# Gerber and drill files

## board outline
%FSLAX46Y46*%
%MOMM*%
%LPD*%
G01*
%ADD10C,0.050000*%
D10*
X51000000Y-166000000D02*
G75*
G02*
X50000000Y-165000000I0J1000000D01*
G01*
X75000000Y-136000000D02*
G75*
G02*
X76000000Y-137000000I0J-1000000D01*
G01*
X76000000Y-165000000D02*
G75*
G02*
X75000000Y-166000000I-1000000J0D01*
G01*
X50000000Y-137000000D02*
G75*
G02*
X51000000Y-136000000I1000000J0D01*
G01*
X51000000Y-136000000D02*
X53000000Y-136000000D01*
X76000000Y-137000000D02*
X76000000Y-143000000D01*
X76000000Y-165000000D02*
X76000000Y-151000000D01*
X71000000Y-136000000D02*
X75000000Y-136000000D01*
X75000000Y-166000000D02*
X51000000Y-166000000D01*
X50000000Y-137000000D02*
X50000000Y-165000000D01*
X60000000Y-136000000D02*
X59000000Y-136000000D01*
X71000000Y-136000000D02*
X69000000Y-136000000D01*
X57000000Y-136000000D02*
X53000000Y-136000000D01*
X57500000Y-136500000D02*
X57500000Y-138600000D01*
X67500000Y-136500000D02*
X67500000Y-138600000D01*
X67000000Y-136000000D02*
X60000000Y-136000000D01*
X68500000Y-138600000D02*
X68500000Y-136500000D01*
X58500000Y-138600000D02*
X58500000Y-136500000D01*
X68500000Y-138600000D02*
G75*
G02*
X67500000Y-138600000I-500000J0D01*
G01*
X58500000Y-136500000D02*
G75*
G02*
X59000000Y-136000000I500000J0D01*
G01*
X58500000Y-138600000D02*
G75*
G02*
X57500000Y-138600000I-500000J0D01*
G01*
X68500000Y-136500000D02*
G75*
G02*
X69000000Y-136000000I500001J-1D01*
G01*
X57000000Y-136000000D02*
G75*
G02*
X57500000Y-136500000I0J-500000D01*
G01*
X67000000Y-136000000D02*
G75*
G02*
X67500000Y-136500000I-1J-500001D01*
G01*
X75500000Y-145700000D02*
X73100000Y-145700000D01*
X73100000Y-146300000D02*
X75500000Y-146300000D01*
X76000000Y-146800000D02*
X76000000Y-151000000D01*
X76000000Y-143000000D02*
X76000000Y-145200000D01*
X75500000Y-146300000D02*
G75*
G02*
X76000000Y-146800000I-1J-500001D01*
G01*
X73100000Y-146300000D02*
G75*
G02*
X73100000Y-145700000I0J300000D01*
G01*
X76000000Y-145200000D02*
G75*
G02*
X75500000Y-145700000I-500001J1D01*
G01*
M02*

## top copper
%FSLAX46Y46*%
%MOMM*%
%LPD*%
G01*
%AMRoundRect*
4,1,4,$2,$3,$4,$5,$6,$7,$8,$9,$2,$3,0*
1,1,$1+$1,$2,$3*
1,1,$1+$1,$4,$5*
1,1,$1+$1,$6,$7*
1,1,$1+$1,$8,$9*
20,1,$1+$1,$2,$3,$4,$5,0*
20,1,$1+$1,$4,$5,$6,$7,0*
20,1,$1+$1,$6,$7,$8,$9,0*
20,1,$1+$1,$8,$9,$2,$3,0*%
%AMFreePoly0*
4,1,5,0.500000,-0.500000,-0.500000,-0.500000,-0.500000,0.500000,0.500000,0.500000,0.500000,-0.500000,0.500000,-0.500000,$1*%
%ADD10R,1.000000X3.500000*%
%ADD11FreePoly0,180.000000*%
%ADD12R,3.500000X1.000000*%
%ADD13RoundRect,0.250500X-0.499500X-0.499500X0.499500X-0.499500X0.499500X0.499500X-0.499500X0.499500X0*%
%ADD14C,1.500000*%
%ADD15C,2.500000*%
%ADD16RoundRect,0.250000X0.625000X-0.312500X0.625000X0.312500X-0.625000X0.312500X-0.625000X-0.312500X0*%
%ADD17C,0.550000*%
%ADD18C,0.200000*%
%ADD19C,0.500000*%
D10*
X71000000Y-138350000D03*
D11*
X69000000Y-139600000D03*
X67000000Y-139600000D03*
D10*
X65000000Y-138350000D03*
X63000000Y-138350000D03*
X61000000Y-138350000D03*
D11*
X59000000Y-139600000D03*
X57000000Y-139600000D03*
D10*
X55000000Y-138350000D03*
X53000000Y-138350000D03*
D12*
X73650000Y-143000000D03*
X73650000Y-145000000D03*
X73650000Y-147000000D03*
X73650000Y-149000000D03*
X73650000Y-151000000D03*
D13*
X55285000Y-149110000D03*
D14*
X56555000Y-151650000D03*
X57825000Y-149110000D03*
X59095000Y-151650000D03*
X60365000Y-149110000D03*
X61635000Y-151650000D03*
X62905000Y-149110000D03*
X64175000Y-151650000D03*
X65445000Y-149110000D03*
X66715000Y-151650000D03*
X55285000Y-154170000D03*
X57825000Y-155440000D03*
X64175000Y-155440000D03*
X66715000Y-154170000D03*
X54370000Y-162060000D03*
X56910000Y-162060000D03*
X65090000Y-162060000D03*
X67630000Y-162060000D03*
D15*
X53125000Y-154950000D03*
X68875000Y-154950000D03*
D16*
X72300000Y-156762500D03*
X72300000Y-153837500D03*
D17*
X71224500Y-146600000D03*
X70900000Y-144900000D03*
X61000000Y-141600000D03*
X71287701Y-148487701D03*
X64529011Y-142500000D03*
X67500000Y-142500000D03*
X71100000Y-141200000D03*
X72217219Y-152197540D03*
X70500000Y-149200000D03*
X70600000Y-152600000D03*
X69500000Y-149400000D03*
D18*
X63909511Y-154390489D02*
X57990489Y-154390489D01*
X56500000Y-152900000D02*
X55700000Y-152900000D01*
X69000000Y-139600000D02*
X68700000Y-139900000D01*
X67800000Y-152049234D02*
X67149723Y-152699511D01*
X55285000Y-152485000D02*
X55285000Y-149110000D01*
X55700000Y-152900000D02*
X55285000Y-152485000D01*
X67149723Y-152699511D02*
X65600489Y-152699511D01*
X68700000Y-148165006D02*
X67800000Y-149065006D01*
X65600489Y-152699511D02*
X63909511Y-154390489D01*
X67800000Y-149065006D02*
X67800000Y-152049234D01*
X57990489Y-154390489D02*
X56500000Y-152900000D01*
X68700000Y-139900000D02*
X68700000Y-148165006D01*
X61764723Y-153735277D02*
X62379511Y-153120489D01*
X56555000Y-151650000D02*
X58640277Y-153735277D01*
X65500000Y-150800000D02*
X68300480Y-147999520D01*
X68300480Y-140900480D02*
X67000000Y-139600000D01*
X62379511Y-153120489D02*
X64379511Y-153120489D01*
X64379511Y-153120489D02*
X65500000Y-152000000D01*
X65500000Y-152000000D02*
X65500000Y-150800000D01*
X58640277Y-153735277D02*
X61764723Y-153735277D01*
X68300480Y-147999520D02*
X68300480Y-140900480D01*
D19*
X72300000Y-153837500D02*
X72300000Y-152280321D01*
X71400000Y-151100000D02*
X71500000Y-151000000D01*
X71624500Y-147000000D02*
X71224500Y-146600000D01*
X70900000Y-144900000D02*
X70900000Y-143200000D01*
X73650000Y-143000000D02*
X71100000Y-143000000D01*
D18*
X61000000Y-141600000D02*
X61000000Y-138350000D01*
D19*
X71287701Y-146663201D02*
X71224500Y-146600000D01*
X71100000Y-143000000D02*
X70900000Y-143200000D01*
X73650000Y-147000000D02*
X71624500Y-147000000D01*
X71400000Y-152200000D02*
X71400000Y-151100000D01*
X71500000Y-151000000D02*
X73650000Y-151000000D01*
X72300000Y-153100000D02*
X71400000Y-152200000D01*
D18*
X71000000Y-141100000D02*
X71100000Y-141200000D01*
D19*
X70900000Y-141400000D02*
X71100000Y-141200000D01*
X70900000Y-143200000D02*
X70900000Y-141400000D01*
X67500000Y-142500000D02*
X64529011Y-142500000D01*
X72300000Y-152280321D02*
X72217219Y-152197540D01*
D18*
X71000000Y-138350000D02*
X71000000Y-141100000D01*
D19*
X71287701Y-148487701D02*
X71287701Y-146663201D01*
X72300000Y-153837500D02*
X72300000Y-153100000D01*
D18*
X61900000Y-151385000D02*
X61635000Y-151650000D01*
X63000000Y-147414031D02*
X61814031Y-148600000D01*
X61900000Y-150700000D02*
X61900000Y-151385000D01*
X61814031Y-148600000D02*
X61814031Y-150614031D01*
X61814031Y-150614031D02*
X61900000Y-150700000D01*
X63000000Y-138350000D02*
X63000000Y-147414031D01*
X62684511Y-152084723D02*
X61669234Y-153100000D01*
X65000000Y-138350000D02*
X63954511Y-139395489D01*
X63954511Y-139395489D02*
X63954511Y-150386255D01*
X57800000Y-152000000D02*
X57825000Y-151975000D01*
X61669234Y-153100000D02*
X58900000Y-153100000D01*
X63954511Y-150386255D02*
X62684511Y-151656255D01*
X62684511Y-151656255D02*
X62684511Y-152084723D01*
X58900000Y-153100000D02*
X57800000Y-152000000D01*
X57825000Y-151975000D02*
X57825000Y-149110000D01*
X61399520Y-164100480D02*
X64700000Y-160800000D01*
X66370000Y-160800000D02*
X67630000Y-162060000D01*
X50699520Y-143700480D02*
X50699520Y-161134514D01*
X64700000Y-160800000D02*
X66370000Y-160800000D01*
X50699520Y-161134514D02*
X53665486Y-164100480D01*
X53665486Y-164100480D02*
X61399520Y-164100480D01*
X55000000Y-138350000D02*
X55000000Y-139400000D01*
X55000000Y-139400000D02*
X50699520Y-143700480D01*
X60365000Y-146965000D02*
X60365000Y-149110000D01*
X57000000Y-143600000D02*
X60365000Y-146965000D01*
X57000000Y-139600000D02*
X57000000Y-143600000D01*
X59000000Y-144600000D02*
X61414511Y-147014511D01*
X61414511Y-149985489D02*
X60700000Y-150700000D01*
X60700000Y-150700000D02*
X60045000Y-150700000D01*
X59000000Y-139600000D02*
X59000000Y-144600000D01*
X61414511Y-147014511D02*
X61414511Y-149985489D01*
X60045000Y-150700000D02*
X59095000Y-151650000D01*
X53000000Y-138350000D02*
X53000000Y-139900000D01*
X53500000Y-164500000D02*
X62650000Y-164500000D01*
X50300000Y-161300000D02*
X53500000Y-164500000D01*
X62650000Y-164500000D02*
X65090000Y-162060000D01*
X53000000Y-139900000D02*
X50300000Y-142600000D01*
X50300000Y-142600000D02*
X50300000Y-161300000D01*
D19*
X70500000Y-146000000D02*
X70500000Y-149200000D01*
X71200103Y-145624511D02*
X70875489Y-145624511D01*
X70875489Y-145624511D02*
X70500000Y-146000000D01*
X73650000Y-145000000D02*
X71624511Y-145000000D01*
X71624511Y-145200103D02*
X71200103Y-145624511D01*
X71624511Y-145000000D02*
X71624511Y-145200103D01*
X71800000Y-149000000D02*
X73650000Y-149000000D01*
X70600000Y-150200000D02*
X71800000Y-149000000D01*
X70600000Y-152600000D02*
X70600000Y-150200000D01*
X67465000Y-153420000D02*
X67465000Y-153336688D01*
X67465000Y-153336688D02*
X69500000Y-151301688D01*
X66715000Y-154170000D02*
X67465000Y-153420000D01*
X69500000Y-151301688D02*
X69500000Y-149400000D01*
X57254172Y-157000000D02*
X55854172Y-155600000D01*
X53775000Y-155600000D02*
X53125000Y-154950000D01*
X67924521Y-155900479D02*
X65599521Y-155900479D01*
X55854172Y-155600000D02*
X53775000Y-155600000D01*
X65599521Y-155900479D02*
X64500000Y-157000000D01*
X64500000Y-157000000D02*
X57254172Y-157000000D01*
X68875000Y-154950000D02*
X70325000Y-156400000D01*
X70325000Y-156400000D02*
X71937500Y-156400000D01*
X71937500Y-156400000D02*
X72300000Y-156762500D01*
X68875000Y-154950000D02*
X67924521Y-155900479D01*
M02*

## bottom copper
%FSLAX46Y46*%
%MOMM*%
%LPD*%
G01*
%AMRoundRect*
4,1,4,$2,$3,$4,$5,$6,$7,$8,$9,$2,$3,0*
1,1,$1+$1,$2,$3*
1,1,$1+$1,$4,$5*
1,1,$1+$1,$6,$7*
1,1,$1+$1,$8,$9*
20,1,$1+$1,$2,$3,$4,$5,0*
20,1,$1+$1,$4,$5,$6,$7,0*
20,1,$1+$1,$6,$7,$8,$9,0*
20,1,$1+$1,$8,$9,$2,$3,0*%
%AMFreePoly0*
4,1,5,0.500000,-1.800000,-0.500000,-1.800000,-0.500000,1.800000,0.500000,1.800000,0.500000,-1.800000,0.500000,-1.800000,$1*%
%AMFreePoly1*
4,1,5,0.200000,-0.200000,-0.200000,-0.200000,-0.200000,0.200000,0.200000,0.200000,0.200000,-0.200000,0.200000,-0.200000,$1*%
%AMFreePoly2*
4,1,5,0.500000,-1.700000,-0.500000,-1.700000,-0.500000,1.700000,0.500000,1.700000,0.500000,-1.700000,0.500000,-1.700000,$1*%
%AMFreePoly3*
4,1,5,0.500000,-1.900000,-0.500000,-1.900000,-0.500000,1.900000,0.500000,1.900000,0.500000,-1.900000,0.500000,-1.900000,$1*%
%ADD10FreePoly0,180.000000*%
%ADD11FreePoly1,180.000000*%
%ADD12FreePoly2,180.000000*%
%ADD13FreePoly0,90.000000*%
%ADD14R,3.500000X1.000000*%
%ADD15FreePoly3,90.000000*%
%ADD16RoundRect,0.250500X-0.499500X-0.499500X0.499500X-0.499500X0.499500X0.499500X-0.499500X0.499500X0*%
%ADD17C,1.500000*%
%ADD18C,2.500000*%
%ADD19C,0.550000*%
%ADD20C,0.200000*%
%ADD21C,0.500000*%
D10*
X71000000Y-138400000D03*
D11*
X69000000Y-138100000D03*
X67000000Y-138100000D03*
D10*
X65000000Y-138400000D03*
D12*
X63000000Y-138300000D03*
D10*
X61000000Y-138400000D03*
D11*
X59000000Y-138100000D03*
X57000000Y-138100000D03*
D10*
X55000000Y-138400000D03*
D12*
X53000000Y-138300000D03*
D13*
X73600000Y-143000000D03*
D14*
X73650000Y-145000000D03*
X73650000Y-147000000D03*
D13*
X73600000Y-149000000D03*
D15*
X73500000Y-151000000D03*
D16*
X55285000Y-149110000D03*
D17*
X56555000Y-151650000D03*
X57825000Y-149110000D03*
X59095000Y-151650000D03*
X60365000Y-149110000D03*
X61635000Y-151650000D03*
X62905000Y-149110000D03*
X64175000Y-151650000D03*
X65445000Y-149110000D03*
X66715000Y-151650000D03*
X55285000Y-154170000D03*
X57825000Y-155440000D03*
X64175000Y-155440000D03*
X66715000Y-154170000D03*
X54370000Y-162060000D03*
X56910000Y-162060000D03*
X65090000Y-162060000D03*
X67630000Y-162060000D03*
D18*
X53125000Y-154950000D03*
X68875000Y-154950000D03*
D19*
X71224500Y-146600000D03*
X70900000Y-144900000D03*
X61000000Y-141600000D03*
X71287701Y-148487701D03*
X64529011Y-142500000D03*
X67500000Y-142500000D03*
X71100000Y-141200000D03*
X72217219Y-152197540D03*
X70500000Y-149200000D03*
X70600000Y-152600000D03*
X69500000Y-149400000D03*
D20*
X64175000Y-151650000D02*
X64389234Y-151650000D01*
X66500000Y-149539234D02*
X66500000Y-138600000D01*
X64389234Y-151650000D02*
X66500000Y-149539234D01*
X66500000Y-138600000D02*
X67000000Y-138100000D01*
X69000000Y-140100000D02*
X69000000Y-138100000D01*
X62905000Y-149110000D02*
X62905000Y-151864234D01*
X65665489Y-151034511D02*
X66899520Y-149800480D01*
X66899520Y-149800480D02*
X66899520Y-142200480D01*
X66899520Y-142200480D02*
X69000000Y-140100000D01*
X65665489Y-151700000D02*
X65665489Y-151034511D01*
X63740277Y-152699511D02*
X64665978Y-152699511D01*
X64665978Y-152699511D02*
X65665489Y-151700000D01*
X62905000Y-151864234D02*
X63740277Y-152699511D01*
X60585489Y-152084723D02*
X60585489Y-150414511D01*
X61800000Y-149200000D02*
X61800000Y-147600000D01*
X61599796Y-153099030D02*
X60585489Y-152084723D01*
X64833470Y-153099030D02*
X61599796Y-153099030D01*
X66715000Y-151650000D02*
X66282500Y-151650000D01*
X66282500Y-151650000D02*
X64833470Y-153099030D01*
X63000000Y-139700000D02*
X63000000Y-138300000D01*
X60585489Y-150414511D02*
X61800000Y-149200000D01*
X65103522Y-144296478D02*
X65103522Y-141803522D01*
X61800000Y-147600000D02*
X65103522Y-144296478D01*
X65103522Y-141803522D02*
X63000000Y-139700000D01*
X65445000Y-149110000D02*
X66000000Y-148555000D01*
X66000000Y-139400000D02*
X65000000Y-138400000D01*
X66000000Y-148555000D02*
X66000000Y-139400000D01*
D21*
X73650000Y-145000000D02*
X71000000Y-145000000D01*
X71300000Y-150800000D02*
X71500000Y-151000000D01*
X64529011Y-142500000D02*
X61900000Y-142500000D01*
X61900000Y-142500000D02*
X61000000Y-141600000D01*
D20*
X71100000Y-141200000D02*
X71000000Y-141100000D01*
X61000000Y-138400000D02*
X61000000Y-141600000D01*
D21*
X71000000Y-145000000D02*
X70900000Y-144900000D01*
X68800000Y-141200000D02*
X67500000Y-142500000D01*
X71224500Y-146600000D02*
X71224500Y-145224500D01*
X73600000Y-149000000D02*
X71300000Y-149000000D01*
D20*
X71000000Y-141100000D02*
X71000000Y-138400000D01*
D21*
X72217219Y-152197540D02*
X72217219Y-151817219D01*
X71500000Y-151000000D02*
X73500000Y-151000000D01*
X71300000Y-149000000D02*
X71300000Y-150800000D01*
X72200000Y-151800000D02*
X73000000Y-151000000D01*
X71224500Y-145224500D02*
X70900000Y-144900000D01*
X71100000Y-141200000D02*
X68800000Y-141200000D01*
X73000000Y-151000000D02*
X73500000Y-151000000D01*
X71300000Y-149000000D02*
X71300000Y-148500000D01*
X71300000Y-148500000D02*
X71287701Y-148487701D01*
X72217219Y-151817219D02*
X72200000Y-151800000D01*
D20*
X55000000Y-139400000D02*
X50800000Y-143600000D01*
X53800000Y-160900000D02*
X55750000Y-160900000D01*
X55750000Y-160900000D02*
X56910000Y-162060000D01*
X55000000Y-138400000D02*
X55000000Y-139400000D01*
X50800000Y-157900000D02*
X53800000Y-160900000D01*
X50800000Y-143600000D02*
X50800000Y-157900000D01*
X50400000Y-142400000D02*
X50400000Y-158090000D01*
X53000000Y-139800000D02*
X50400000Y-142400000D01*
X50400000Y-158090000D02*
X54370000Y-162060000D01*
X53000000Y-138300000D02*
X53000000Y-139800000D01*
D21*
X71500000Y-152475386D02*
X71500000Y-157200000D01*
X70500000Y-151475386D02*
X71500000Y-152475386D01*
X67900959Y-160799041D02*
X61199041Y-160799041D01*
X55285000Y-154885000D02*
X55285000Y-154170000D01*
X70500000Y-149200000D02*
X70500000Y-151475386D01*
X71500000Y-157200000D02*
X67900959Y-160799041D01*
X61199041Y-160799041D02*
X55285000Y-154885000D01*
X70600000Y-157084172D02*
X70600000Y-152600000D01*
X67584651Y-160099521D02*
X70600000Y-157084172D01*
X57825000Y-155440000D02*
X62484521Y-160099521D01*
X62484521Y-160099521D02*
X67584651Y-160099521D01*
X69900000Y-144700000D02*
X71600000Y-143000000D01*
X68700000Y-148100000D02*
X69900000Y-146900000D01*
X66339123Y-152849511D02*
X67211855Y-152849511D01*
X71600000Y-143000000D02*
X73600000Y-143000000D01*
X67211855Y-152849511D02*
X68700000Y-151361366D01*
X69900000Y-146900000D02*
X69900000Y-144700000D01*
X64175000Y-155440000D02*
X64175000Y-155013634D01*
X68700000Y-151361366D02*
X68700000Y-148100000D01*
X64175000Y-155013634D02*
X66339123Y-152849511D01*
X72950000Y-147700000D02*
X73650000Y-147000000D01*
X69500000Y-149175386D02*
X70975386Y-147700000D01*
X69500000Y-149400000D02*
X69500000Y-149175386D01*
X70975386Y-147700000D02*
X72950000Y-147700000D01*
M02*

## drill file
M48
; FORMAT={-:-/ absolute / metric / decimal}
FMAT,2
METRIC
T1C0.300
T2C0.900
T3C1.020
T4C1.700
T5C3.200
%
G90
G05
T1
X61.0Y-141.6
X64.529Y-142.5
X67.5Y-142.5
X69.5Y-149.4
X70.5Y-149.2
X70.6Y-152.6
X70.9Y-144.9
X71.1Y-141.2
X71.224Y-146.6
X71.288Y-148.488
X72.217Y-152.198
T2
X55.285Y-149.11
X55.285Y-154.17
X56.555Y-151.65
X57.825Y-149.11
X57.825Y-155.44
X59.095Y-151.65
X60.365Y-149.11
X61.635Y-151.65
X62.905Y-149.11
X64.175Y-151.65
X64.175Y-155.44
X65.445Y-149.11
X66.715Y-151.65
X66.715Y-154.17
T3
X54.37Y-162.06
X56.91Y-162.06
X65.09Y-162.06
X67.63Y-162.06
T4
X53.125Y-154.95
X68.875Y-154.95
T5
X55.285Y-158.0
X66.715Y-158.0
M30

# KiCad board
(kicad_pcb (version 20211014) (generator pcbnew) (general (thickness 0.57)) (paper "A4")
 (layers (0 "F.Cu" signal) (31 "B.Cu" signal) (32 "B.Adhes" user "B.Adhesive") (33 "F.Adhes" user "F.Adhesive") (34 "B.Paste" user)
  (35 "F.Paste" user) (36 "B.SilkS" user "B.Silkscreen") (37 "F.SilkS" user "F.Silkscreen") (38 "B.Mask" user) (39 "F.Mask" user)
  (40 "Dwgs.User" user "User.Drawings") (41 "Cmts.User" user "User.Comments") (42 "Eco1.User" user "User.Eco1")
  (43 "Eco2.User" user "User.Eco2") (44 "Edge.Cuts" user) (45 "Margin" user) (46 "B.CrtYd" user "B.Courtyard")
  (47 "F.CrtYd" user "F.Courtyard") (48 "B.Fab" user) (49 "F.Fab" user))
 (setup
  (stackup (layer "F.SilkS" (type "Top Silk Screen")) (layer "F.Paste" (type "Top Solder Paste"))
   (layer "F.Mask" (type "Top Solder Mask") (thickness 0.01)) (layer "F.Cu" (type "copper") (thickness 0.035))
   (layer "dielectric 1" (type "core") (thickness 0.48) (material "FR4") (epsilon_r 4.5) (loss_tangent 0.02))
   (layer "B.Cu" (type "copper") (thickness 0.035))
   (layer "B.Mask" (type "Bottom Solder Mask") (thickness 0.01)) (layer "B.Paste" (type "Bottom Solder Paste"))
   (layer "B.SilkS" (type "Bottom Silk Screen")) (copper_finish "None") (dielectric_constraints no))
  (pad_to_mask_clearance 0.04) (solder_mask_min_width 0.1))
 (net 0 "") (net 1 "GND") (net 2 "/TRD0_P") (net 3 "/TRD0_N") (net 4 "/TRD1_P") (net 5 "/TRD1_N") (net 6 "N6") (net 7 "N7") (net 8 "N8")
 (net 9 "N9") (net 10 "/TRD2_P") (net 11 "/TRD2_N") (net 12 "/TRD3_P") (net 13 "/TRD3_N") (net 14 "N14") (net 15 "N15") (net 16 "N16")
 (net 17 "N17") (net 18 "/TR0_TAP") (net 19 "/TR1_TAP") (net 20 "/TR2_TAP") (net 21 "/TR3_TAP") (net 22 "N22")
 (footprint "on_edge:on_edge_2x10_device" (layer "F.Cu") (at 67 136 180)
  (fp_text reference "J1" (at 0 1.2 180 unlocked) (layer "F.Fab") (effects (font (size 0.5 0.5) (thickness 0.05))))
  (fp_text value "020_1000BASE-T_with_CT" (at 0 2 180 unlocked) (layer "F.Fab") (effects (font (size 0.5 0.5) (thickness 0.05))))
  (fp_line (start 7 0) (end 8 0) (layer "Edge.Cuts") (width 0.05))
  (fp_line (start -4 0) (end -2 0) (layer "Edge.Cuts") (width 0.05))
  (fp_line (start 10 0) (end 14 0) (layer "Edge.Cuts") (width 0.05))
  (fp_line (start 9.5 -0.5) (end 9.5 -2.6) (layer "Edge.Cuts") (width 0.05))
  (fp_line (start -0.5 -0.5) (end -0.5 -2.6) (layer "Edge.Cuts") (width 0.05))
  (fp_line (start 0 0) (end 7 0) (layer "Edge.Cuts") (width 0.05))
  (fp_line (start -1.5 -2.6) (end -1.5 -0.5) (layer "Edge.Cuts") (width 0.05))
  (fp_line (start 8.5 -2.6) (end 8.5 -0.5) (layer "Edge.Cuts") (width 0.05))
  (fp_arc (start -1.5 -2.6) (mid -1 -3.1) (end -0.5 -2.6) (layer "Edge.Cuts") (width 0.05))
  (fp_arc (start 8.5 -0.5) (mid 8.353553 -0.146447) (end 8 0) (layer "Edge.Cuts") (width 0.05))
  (fp_arc (start 8.5 -2.6) (mid 9 -3.1) (end 9.5 -2.6) (layer "Edge.Cuts") (width 0.05))
  (fp_arc (start -1.5 -0.5) (mid -1.646447 -0.146447) (end -2 0) (layer "Edge.Cuts") (width 0.05))
  (fp_arc (start 10 0) (mid 9.646447 -0.146447) (end 9.5 -0.5) (layer "Edge.Cuts") (width 0.05))
  (fp_arc (start 0 0) (mid -0.353553 -0.146447) (end -0.5 -0.5) (layer "Edge.Cuts") (width 0.05))
  (pad "1" smd rect locked (at -4 -2.35) (size 1 3.5) (layers "F.Cu" "F.Mask") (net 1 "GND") (zone_connect 0))
  (pad "2" smd custom locked (at -2 -3.6 180) (size 1 1) (layers "F.Cu" "F.Mask") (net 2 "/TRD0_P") (zone_connect 0)
   (options (clearance outline) (anchor rect)) (primitives))
  (pad "3" smd custom locked (at 0 -3.6 180) (size 1 1) (layers "F.Cu" "F.Mask") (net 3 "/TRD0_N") (zone_connect 0)
   (options (clearance outline) (anchor rect)) (primitives))
  (pad "4" smd rect locked (at 2 -2.35) (size 1 3.5) (layers "F.Cu" "F.Mask") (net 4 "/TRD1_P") (zone_connect 0))
  (pad "5" smd rect locked (at 4 -2.35) (size 1 3.5) (layers "F.Cu" "F.Mask") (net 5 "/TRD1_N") (zone_connect 0))
  (pad "6" smd rect locked (at 6 -2.35) (size 1 3.5) (layers "F.Cu" "F.Mask") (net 1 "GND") (zone_connect 0))
  (pad "7" smd custom locked (at 8 -3.6 180) (size 1 1) (layers "F.Cu" "F.Mask") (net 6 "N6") (zone_connect 0)
   (options (clearance outline) (anchor rect)) (primitives))
  (pad "8" smd custom locked (at 10 -3.6 180) (size 1 1) (layers "F.Cu" "F.Mask") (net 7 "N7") (zone_connect 0)
   (options (clearance outline) (anchor rect)) (primitives))
  (pad "9" smd rect locked (at 12 -2.35) (size 1 3.5) (layers "F.Cu" "F.Mask") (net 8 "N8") (zone_connect 0))
  (pad "10" smd rect locked (at 14 -2.35) (size 1 3.5) (layers "F.Cu" "F.Mask") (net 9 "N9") (zone_connect 0))
  (pad "11" smd custom locked (at -4 -2.4 180) (size 1 3.6) (layers "B.Cu" "B.Mask") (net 1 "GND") (zone_connect 0)
   (options (clearance outline) (anchor rect)) (primitives))
  (pad "12" smd custom locked (at -2 -2.1 180) (size 0.4 0.4) (layers "B.Cu" "B.Mask") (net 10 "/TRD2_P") (zone_connect 0)
   (options (clearance outline) (anchor rect)) (primitives))
  (pad "13" smd custom locked (at 0 -2.1 180) (size 0.4 0.4) (layers "B.Cu" "B.Mask") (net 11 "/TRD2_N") (zone_connect 0)
   (options (clearance outline) (anchor rect)) (primitives))
  (pad "14" smd custom locked (at 2 -2.4 180) (size 1 3.6) (layers "B.Cu" "B.Mask") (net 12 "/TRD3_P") (zone_connect 0)
   (options (clearance outline) (anchor rect)) (primitives))
  (pad "15" smd custom locked (at 4 -2.3 180) (size 1 3.4) (layers "B.Cu" "B.Mask") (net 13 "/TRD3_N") (zone_connect 0)
   (options (clearance outline) (anchor rect)) (primitives))
  (pad "16" smd custom locked (at 6 -2.4 180) (size 1 3.6) (layers "B.Cu" "B.Mask") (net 1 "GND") (zone_connect 0)
   (options (clearance outline) (anchor rect)) (primitives))
  (pad "17" smd custom locked (at 8 -2.1 180) (size 0.4 0.4) (layers "B.Cu" "B.Mask") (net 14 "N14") (zone_connect 0)
   (options (clearance outline) (anchor rect)) (primitives))
  (pad "18" smd custom locked (at 10 -2.1 180) (size 0.4 0.4) (layers "B.Cu" "B.Mask") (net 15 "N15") (zone_connect 0)
   (options (clearance outline) (anchor rect)) (primitives))
  (pad "19" smd custom locked (at 12 -2.4 180) (size 1 3.6) (layers "B.Cu" "B.Mask") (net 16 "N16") (zone_connect 0)
   (options (clearance outline) (anchor rect)) (primitives))
  (pad "20" smd custom locked (at 14 -2.3 180) (size 1 3.4) (layers "B.Cu" "B.Mask") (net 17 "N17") (zone_connect 0)
   (options (clearance outline) (anchor rect)) (primitives)))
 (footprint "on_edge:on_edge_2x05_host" (layer "F.Cu") (at 76 147 -90)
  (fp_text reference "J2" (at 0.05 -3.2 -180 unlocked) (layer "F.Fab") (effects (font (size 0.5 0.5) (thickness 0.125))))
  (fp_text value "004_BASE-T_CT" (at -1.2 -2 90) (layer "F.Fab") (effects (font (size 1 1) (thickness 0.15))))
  (fp_line (start -1.3 0.5) (end -1.3 2.9) (layer "Edge.Cuts") (width 0.05))
  (fp_line (start -0.7 2.9) (end -0.7 0.5) (layer "Edge.Cuts") (width 0.05))
  (fp_line (start -0.2 0) (end 4 0) (layer "Edge.Cuts") (width 0.05))
  (fp_line (start -4 0) (end -1.8 0) (layer "Edge.Cuts") (width 0.05))
  (fp_arc (start -0.7 0.5) (mid -0.553553 0.146447) (end -0.2 0) (layer "Edge.Cuts") (width 0.05))
  (fp_arc (start -0.7 2.9) (mid -1 3.2) (end -1.3 2.9) (layer "Edge.Cuts") (width 0.05))
  (fp_arc (start -1.8 0) (mid -1.446447 0.146447) (end -1.3 0.5) (layer "Edge.Cuts") (width 0.05))
  (pad "1" smd rect (at -4 2.35 270) (size 1 3.5) (layers "F.Cu" "F.Mask") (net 1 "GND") (zone_connect 0))
  (pad "2" smd rect (at -2 2.35 270) (size 1 3.5) (layers "F.Cu" "F.Mask") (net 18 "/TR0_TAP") (zone_connect 0))
  (pad "3" smd rect (at 0 2.35 270) (size 1 3.5) (layers "F.Cu" "F.Mask") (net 1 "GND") (zone_connect 0))
  (pad "4" smd rect (at 2 2.35 270) (size 1 3.5) (layers "F.Cu" "F.Mask") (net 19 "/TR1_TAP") (zone_connect 0))
  (pad "5" smd rect (at 4 2.35 270) (size 1 3.5) (layers "F.Cu" "F.Mask") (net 1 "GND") (zone_connect 0))
  (pad "6" smd custom (at -4 2.4 90) (size 1 3.6) (layers "B.Cu" "B.Mask") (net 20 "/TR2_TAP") (zone_connect 0)
   (options (clearance outline) (anchor rect)) (primitives))
  (pad "7" smd rect (at -2 2.35 90) (size 1 3.5) (layers "B.Cu" "B.Mask") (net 1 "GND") (zone_connect 0))
  (pad "8" smd rect (at 0 2.35 90) (size 1 3.5) (layers "B.Cu" "B.Mask") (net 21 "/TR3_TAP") (zone_connect 0))
  (pad "9" smd custom (at 2 2.4 90) (size 1 3.6) (layers "B.Cu" "B.Mask") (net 1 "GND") (zone_connect 0)
   (options (clearance outline) (anchor rect)) (primitives))
  (pad "10" smd custom (at 4 2.5 90) (size 1 3.8) (layers "B.Cu" "B.Mask") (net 1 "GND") (zone_connect 0)
   (options (clearance outline) (anchor rect)) (primitives)))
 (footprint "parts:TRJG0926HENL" (layer "F.Cu") (at 61 158)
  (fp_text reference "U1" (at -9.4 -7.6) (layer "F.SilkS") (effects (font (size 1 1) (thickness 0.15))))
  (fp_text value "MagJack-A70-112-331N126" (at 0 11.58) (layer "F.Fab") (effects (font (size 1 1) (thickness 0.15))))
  (pad "" np_thru_hole circle locked (at -5.715 0) (size 3.2 3.2) (drill 3.2) (layers *.Cu *.Mask))
  (pad "" np_thru_hole circle locked (at 5.715 0) (size 3.2 3.2) (drill 3.2) (layers *.Cu *.Mask))
  (pad "1" thru_hole roundrect locked (at -5.715 -8.89) (size 1.5 1.5) (drill 0.9) (layers *.Cu *.Mask) (roundrect_rratio 0.167)
   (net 2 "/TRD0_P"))
  (pad "2" thru_hole circle locked (at -4.445 -6.35) (size 1.5 1.5) (drill 0.9) (layers *.Cu *.Mask) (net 3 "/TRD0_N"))
  (pad "3" thru_hole circle locked (at -3.175 -8.89) (size 1.5 1.5) (drill 0.9) (layers *.Cu *.Mask) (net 4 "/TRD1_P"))
  (pad "4" thru_hole circle locked (at -1.905 -6.35) (size 1.5 1.5) (drill 0.9) (layers *.Cu *.Mask) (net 6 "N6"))
  (pad "5" thru_hole circle locked (at -0.635 -8.89) (size 1.5 1.5) (drill 0.9) (layers *.Cu *.Mask) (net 7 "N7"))
  (pad "6" thru_hole circle locked (at 0.635 -6.35 90) (size 1.5 1.5) (drill 0.9) (layers *.Cu *.Mask) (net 5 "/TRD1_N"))
  (pad "7" thru_hole circle locked (at 1.905 -8.89) (size 1.5 1.5) (drill 0.9) (layers *.Cu *.Mask) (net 10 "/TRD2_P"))
  (pad "8" thru_hole circle locked (at 3.175 -6.35) (size 1.5 1.5) (drill 0.9) (layers *.Cu *.Mask) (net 11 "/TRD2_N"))
  (pad "9" thru_hole circle locked (at 4.445 -8.89) (size 1.5 1.5) (drill 0.9) (layers *.Cu *.Mask) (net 12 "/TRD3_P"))
  (pad "10" thru_hole circle locked (at 5.715 -6.35) (size 1.5 1.5) (drill 0.9) (layers *.Cu *.Mask) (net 13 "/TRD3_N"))
  (pad "11" thru_hole circle locked (at -5.715 -3.83) (size 1.5 1.5) (drill 0.9) (layers *.Cu *.Mask) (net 18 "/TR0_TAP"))
  (pad "12" thru_hole circle locked (at -3.175 -2.56) (size 1.5 1.5) (drill 0.9) (layers *.Cu *.Mask) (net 19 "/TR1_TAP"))
  (pad "13" thru_hole circle locked (at 3.175 -2.56) (size 1.5 1.5) (drill 0.9) (layers *.Cu *.Mask) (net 20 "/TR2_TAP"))
  (pad "14" thru_hole circle locked (at 5.715 -3.83) (size 1.5 1.5) (drill 0.9) (layers *.Cu *.Mask) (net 21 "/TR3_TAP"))
  (pad "15" thru_hole circle locked (at -6.63 4.06) (size 1.5 1.5) (drill 1.02) (layers *.Cu *.Mask) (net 17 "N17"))
  (pad "16" thru_hole circle locked (at -4.09 4.06) (size 1.5 1.5) (drill 1.02) (layers *.Cu *.Mask) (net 16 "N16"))
  (pad "17" thru_hole circle locked (at 4.09 4.06) (size 1.5 1.5) (drill 1.02) (layers *.Cu *.Mask) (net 9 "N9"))
  (pad "18" thru_hole circle locked (at 6.63 4.06) (size 1.5 1.5) (drill 1.02) (layers *.Cu *.Mask) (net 8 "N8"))
  (pad "19" thru_hole circle locked (at -7.875 -3.05) (size 2.5 2.5) (drill 1.7) (layers *.Cu *.Mask) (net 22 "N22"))
  (pad "20" thru_hole circle locked (at 7.875 -3.05) (size 2.5 2.5) (drill 1.7) (layers *.Cu *.Mask) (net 22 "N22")))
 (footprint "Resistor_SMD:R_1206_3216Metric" (layer "F.Cu") (at 72.3 155.3 90)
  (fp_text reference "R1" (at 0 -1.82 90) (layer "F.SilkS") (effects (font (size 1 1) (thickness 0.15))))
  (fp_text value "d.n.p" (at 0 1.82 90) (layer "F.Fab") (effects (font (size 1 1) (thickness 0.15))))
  (pad "1" smd roundrect (at -1.4625 0 90) (size 1.125 1.75) (layers "F.Cu" "F.Paste" "F.Mask") (roundrect_rratio 0.222222) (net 22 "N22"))
  (pad "2" smd roundrect (at 1.4625 0 90) (size 1.125 1.75) (layers "F.Cu" "F.Paste" "F.Mask") (roundrect_rratio 0.222222) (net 1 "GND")))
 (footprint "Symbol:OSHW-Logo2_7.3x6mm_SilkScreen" (layer "B.Cu") (at 72 162 180)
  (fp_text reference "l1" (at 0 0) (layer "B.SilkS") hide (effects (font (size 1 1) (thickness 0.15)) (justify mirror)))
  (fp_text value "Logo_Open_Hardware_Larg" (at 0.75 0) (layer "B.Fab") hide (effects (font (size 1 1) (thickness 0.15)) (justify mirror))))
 (gr_arc (start 51 166) (mid 50.292893 165.707107) (end 50 165) (layer "Edge.Cuts") (width 0.05))
 (gr_arc (start 75 136) (mid 75.707107 136.292893) (end 76 137) (layer "Edge.Cuts") (width 0.05))
 (gr_arc (start 76 165) (mid 75.707107 165.707107) (end 75 166) (layer "Edge.Cuts") (width 0.05))
 (gr_arc (start 50 137) (mid 50.292893 136.292893) (end 51 136) (layer "Edge.Cuts") (width 0.05))
 (gr_line (start 51 136) (end 53 136) (layer "Edge.Cuts") (width 0.05))
 (gr_line (start 76 137) (end 76 143) (layer "Edge.Cuts") (width 0.05))
 (gr_line (start 76 165) (end 76 151) (layer "Edge.Cuts") (width 0.05))
 (gr_line (start 71 136) (end 75 136) (layer "Edge.Cuts") (width 0.05))
 (gr_line (start 75 166) (end 51 166) (layer "Edge.Cuts") (width 0.05))
 (gr_line (start 50 137) (end 50 165) (layer "Edge.Cuts") (width 0.05))
 (segment (start 63.909511 154.390489) (end 57.990489 154.390489) (width 0.2) (layer "F.Cu") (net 2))
 (segment (start 56.5 152.9) (end 55.7 152.9) (width 0.2) (layer "F.Cu") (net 2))
 (segment (start 69 139.6) (end 68.7 139.9) (width 0.2) (layer "F.Cu") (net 2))
 (segment (start 67.8 152.049234) (end 67.149723 152.699511) (width 0.2) (layer "F.Cu") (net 2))
 (segment (start 55.285 152.485) (end 55.285 149.11) (width 0.2) (layer "F.Cu") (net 2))
 (segment (start 55.7 152.9) (end 55.285 152.485) (width 0.2) (layer "F.Cu") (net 2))
 (segment (start 67.149723 152.699511) (end 65.600489 152.699511) (width 0.2) (layer "F.Cu") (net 2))
 (segment (start 68.7 148.165006) (end 67.8 149.065006) (width 0.2) (layer "F.Cu") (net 2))
 (segment (start 65.600489 152.699511) (end 63.909511 154.390489) (width 0.2) (layer "F.Cu") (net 2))
 (segment (start 67.8 149.065006) (end 67.8 152.049234) (width 0.2) (layer "F.Cu") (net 2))
 (segment (start 57.990489 154.390489) (end 56.5 152.9) (width 0.2) (layer "F.Cu") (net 2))
 (segment (start 68.7 139.9) (end 68.7 148.165006) (width 0.2) (layer "F.Cu") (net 2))
 (segment (start 61.764723 153.735277) (end 62.379511 153.120489) (width 0.2) (layer "F.Cu") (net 3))
 (segment (start 56.555 151.65) (end 58.640277 153.735277) (width 0.2) (layer "F.Cu") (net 3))
 (segment (start 65.5 150.8) (end 68.30048 147.99952) (width 0.2) (layer "F.Cu") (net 3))
 (segment (start 68.30048 140.90048) (end 67 139.6) (width 0.2) (layer "F.Cu") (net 3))
 (segment (start 62.379511 153.120489) (end 64.379511 153.120489) (width 0.2) (layer "F.Cu") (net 3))
 (segment (start 64.379511 153.120489) (end 65.5 152) (width 0.2) (layer "F.Cu") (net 3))
 (segment (start 65.5 152) (end 65.5 150.8) (width 0.2) (layer "F.Cu") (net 3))
 (segment (start 58.640277 153.735277) (end 61.764723 153.735277) (width 0.2) (layer "F.Cu") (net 3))
 (segment (start 68.30048 147.99952) (end 68.30048 140.90048) (width 0.2) (layer "F.Cu") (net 3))
 (segment (start 64.175 151.65) (end 64.389234 151.65) (width 0.2) (layer "B.Cu") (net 11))
 (segment (start 66.5 149.539234) (end 66.5 138.6) (width 0.2) (layer "B.Cu") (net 11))
 (segment (start 64.389234 151.65) (end 66.5 149.539234) (width 0.2) (layer "B.Cu") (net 11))
 (segment (start 66.5 138.6) (end 67 138.1) (width 0.2) (layer "B.Cu") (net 11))
 (segment (start 69 140.1) (end 69 138.1) (width 0.2) (layer "B.Cu") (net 10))
 (segment (start 62.905 149.11) (end 62.905 151.864234) (width 0.2) (layer "B.Cu") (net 10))
 (segment (start 65.665489 151.034511) (end 66.89952 149.80048) (width 0.2) (layer "B.Cu") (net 10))
 (segment (start 66.89952 149.80048) (end 66.89952 142.20048) (width 0.2) (layer "B.Cu") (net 10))
 (segment (start 66.89952 142.20048) (end 69 140.1) (width 0.2) (layer "B.Cu") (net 10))
 (segment (start 65.665489 151.7) (end 65.665489 151.034511) (width 0.2) (layer "B.Cu") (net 10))
 (segment (start 63.740277 152.699511) (end 64.665978 152.699511) (width 0.2) (layer "B.Cu") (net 10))
 (segment (start 64.665978 152.699511) (end 65.665489 151.7) (width 0.2) (layer "B.Cu") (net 10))
 (segment (start 62.905 151.864234) (end 63.740277 152.699511) (width 0.2) (layer "B.Cu") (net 10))
 (segment (start 60.585489 152.084723) (end 60.585489 150.414511) (width 0.2) (layer "B.Cu") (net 13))
 (segment (start 61.8 149.2) (end 61.8 147.6) (width 0.2) (layer "B.Cu") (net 13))
 (segment (start 61.599796 153.09903) (end 60.585489 152.084723) (width 0.2) (layer "B.Cu") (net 13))
 (segment (start 64.83347 153.09903) (end 61.599796 153.09903) (width 0.2) (layer "B.Cu") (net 13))
 (segment (start 66.715 151.65) (end 66.2825 151.65) (width 0.2) (layer "B.Cu") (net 13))
 (segment (start 66.2825 151.65) (end 64.83347 153.09903) (width 0.2) (layer "B.Cu") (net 13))
 (segment (start 63 139.7) (end 63 138.3) (width 0.2) (layer "B.Cu") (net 13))
 (segment (start 60.585489 150.414511) (end 61.8 149.2) (width 0.2) (layer "B.Cu") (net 13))
 (segment (start 65.103522 144.296478) (end 65.103522 141.803522) (width 0.2) (layer "B.Cu") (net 13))
 (segment (start 61.8 147.6) (end 65.103522 144.296478) (width 0.2) (layer "B.Cu") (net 13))
 (segment (start 65.103522 141.803522) (end 63 139.7) (width 0.2) (layer "B.Cu") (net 13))
 (segment (start 65.445 149.11) (end 66 148.555) (width 0.2) (layer "B.Cu") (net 12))
 (segment (start 66 139.4) (end 65 138.4) (width 0.2) (layer "B.Cu") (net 12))
 (segment (start 66 148.555) (end 66 139.4) (width 0.2) (layer "B.Cu") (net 12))
 (segment (start 72.3 153.8375) (end 72.3 152.280321) (width 0.5) (layer "F.Cu") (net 1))
 (segment (start 71.4 151.1) (end 71.5 151) (width 0.5) (layer "F.Cu") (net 1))
 (segment (start 71.6245 147) (end 71.2245 146.6) (width 0.5) (layer "F.Cu") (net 1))
 (segment (start 70.9 144.9) (end 70.9 143.2) (width 0.5) (layer "F.Cu") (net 1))
 (segment (start 73.65 143) (end 71.1 143) (width 0.5) (layer "F.Cu") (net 1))
 (segment (start 61 141.6) (end 61 138.35) (width 0.2) (layer "F.Cu") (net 1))
 (segment (start 71.287701 146.663201) (end 71.2245 146.6) (width 0.5) (layer "F.Cu") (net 1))
 (segment (start 71.1 143) (end 70.9 143.2) (width 0.5) (layer "F.Cu") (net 1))
 (segment (start 73.65 147) (end 71.6245 147) (width 0.5) (layer "F.Cu") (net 1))
 (segment (start 71.4 152.2) (end 71.4 151.1) (width 0.5) (layer "F.Cu") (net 1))
 (segment (start 71.5 151) (end 73.65 151) (width 0.5) (layer "F.Cu") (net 1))
 (segment (start 72.3 153.1) (end 71.4 152.2) (width 0.5) (layer "F.Cu") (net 1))
 (segment (start 71 141.1) (end 71.1 141.2) (width 0.2) (layer "F.Cu") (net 1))
 (segment (start 70.9 141.4) (end 71.1 141.2) (width 0.5) (layer "F.Cu") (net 1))
 (segment (start 70.9 143.2) (end 70.9 141.4) (width 0.5) (layer "F.Cu") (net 1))
 (segment (start 67.5 142.5) (end 64.529011 142.5) (width 0.5) (layer "F.Cu") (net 1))
 (segment (start 72.3 152.280321) (end 72.217219 152.19754) (width 0.5) (layer "F.Cu") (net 1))
 (segment (start 71 138.35) (end 71 141.1) (width 0.2) (layer "F.Cu") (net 1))
 (segment (start 71.287701 148.487701) (end 71.287701 146.663201) (width 0.5) (layer "F.Cu") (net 1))
 (segment (start 72.3 153.8375) (end 72.3 153.1) (width 0.5) (layer "F.Cu") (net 1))
 (via (at 71.2245 146.6) (size 0.55) (drill 0.3) (layers "F.Cu" "B.Cu") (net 1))
 (via (at 70.9 144.9) (size 0.55) (drill 0.3) (layers "F.Cu" "B.Cu") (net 1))
 (via (at 61 141.6) (size 0.55) (drill 0.3) (layers "F.Cu" "B.Cu") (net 1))
 (via (at 71.287701 148.487701) (size 0.55) (drill 0.3) (layers "F.Cu" "B.Cu") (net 1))
 (via (at 64.529011 142.5) (size 0.55) (drill 0.3) (layers "F.Cu" "B.Cu") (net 1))
 (via (at 67.5 142.5) (size 0.55) (drill 0.3) (layers "F.Cu" "B.Cu") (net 1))
 (via (at 71.1 141.2) (size 0.55) (drill 0.3) (layers "F.Cu" "B.Cu") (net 1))
 (via (at 72.217219 152.19754) (size 0.55) (drill 0.3) (layers "F.Cu" "B.Cu") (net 1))
 (segment (start 73.65 145) (end 71 145) (width 0.5) (layer "B.Cu") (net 1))
 (segment (start 71.3 150.8) (end 71.5 151) (width 0.5) (layer "B.Cu") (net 1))
 (segment (start 64.529011 142.5) (end 61.9 142.5) (width 0.5) (layer "B.Cu") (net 1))
 (segment (start 61.9 142.5) (end 61 141.6) (width 0.5) (layer "B.Cu") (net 1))
 (segment (start 71.1 141.2) (end 71 141.1) (width 0.2) (layer "B.Cu") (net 1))
 (segment (start 61 138.4) (end 61 141.6) (width 0.2) (layer "B.Cu") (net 1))
 (segment (start 71 145) (end 70.9 144.9) (width 0.5) (layer "B.Cu") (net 1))
 (segment (start 68.8 141.2) (end 67.5 142.5) (width 0.5) (layer "B.Cu") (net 1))
 (segment (start 71.2245 146.6) (end 71.2245 145.2245) (width 0.5) (layer "B.Cu") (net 1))
 (segment (start 73.6 149) (end 71.3 149) (width 0.5) (layer "B.Cu") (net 1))
 (segment (start 71 141.1) (end 71 138.4) (width 0.2) (layer "B.Cu") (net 1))
 (segment (start 72.217219 152.19754) (end 72.217219 151.817219) (width 0.5) (layer "B.Cu") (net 1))
 (segment (start 71.5 151) (end 73.5 151) (width 0.5) (layer "B.Cu") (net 1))
 (segment (start 71.3 149) (end 71.3 150.8) (width 0.5) (layer "B.Cu") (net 1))
 (segment (start 72.2 151.8) (end 73 151) (width 0.5) (layer "B.Cu") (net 1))
 (segment (start 71.2245 145.2245) (end 70.9 144.9) (width 0.5) (layer "B.Cu") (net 1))
 (segment (start 71.1 141.2) (end 68.8 141.2) (width 0.5) (layer "B.Cu") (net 1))
 (segment (start 73 151) (end 73.5 151) (width 0.5) (layer "B.Cu") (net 1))
 (segment (start 71.3 149) (end 71.3 148.5) (width 0.5) (layer "B.Cu") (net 1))
 (segment (start 71.3 148.5) (end 71.287701 148.487701) (width 0.5) (layer "B.Cu") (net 1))
 (segment (start 72.217219 151.817219) (end 72.2 151.8) (width 0.5) (layer "B.Cu") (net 1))
 (segment (start 61.9 151.385) (end 61.635 151.65) (width 0.2) (layer "F.Cu") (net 5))
 (segment (start 63 147.414031) (end 61.814031 148.6) (width 0.2) (layer "F.Cu") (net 5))
 (segment (start 61.9 150.7) (end 61.9 151.385) (width 0.2) (layer "F.Cu") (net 5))
 (segment (start 61.814031 148.6) (end 61.814031 150.614031) (width 0.2) (layer "F.Cu") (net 5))
 (segment (start 61.814031 150.614031) (end 61.9 150.7) (width 0.2) (layer "F.Cu") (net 5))
 (segment (start 63 138.35) (end 63 147.414031) (width 0.2) (layer "F.Cu") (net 5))
 (segment (start 62.684511 152.084723) (end 61.669234 153.1) (width 0.2) (layer "F.Cu") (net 4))
 (segment (start 65 138.35) (end 63.954511 139.395489) (width 0.2) (layer "F.Cu") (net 4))
 (segment (start 63.954511 139.395489) (end 63.954511 150.386255) (width 0.2) (layer "F.Cu") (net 4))
 (segment (start 57.8 152) (end 57.825 151.975) (width 0.2) (layer "F.Cu") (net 4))
 (segment (start 61.669234 153.1) (end 58.9 153.1) (width 0.2) (layer "F.Cu") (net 4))
 (segment (start 63.954511 150.386255) (end 62.684511 151.656255) (width 0.2) (layer "F.Cu") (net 4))
 (segment (start 62.684511 151.656255) (end 62.684511 152.084723) (width 0.2) (layer "F.Cu") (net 4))
 (segment (start 58.9 153.1) (end 57.8 152) (width 0.2) (layer "F.Cu") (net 4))
 (segment (start 57.825 151.975) (end 57.825 149.11) (width 0.2) (layer "F.Cu") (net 4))
 (segment (start 55 139.4) (end 50.8 143.6) (width 0.2) (layer "B.Cu") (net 16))
 (segment (start 53.8 160.9) (end 55.75 160.9) (width 0.2) (layer "B.Cu") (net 16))
 (segment (start 55.75 160.9) (end 56.91 162.06) (width 0.2) (layer "B.Cu") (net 16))
 (segment (start 55 138.4) (end 55 139.4) (width 0.2) (layer "B.Cu") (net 16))
 (segment (start 50.8 157.9) (end 53.8 160.9) (width 0.2) (layer "B.Cu") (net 16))
 (segment (start 50.8 143.6) (end 50.8 157.9) (width 0.2) (layer "B.Cu") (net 16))
 (segment (start 61.39952 164.10048) (end 64.7 160.8) (width 0.2) (layer "F.Cu") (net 8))
 (segment (start 66.37 160.8) (end 67.63 162.06) (width 0.2) (layer "F.Cu") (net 8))
 (segment (start 50.69952 143.70048) (end 50.69952 161.134514) (width 0.2) (layer "F.Cu") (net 8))
 (segment (start 64.7 160.8) (end 66.37 160.8) (width 0.2) (layer "F.Cu") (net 8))
 (segment (start 50.69952 161.134514) (end 53.665486 164.10048) (width 0.2) (layer "F.Cu") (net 8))
 (segment (start 53.665486 164.10048) (end 61.39952 164.10048) (width 0.2) (layer "F.Cu") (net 8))
 (segment (start 55 138.35) (end 55 139.4) (width 0.2) (layer "F.Cu") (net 8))
 (segment (start 55 139.4) (end 50.69952 143.70048) (width 0.2) (layer "F.Cu") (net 8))
 (segment (start 60.365 146.965) (end 60.365 149.11) (width 0.2) (layer "F.Cu") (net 7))
 (segment (start 57 143.6) (end 60.365 146.965) (width 0.2) (layer "F.Cu") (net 7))
 (segment (start 57 139.6) (end 57 143.6) (width 0.2) (layer "F.Cu") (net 7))
 (segment (start 59 144.6) (end 61.414511 147.014511) (width 0.2) (layer "F.Cu") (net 6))
 (segment (start 61.414511 149.985489) (end 60.7 150.7) (width 0.2) (layer "F.Cu") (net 6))
 (segment (start 60.7 150.7) (end 60.045 150.7) (width 0.2) (layer "F.Cu") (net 6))
 (segment (start 59 139.6) (end 59 144.6) (width 0.2) (layer "F.Cu") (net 6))
 (segment (start 61.414511 147.014511) (end 61.414511 149.985489) (width 0.2) (layer "F.Cu") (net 6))
 (segment (start 60.045 150.7) (end 59.095 151.65) (width 0.2) (layer "F.Cu") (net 6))
 (segment (start 50.4 142.4) (end 50.4 158.09) (width 0.2) (layer "B.Cu") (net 17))
 (segment (start 53 139.8) (end 50.4 142.4) (width 0.2) (layer "B.Cu") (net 17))
 (segment (start 50.4 158.09) (end 54.37 162.06) (width 0.2) (layer "B.Cu") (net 17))
 (segment (start 53 138.3) (end 53 139.8) (width 0.2) (layer "B.Cu") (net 17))
 (segment (start 53 138.35) (end 53 139.9) (width 0.2) (layer "F.Cu") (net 9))
 (segment (start 53.5 164.5) (end 62.65 164.5) (width 0.2) (layer "F.Cu") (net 9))
 (segment (start 50.3 161.3) (end 53.5 164.5) (width 0.2) (layer "F.Cu") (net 9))
 (segment (start 62.65 164.5) (end 65.09 162.06) (width 0.2) (layer "F.Cu") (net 9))
 (segment (start 53 139.9) (end 50.3 142.6) (width 0.2) (layer "F.Cu") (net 9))
 (segment (start 50.3 142.6) (end 50.3 161.3) (width 0.2) (layer "F.Cu") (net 9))
 (segment (start 70.5 146) (end 70.5 149.2) (width 0.5) (layer "F.Cu") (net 18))
 (segment (start 71.200103 145.624511) (end 70.875489 145.624511) (width 0.5) (layer "F.Cu") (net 18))
 (segment (start 70.875489 145.624511) (end 70.5 146) (width 0.5) (layer "F.Cu") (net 18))
 (segment (start 73.65 145) (end 71.624511 145) (width 0.5) (layer "F.Cu") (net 18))
 (segment (start 71.624511 145.200103) (end 71.200103 145.624511) (width 0.5) (layer "F.Cu") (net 18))
 (segment (start 71.624511 145) (end 71.624511 145.200103) (width 0.5) (layer "F.Cu") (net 18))
 (via (at 70.5 149.2) (size 0.55) (drill 0.3) (layers "F.Cu" "B.Cu") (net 18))
 (segment (start 71.5 152.475386) (end 71.5 157.2) (width 0.5) (layer "B.Cu") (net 18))
 (segment (start 70.5 151.475386) (end 71.5 152.475386) (width 0.5) (layer "B.Cu") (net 18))
 (segment (start 67.900959 160.799041) (end 61.199041 160.799041) (width 0.5) (layer "B.Cu") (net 18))
 (segment (start 55.285 154.885) (end 55.285 154.17) (width 0.5) (layer "B.Cu") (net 18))
 (segment (start 70.5 149.2) (end 70.5 151.475386) (width 0.5) (layer "B.Cu") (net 18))
 (segment (start 71.5 157.2) (end 67.900959 160.799041) (width 0.5) (layer "B.Cu") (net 18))
 (segment (start 61.199041 160.799041) (end 55.285 154.885) (width 0.5) (layer "B.Cu") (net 18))
 (segment (start 71.8 149) (end 73.65 149) (width 0.5) (layer "F.Cu") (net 19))
 (segment (start 70.6 150.2) (end 71.8 149) (width 0.5) (layer "F.Cu") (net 19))
 (segment (start 70.6 152.6) (end 70.6 150.2) (width 0.5) (layer "F.Cu") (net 19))
 (via (at 70.6 152.6) (size 0.55) (drill 0.3) (layers "F.Cu" "B.Cu") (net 19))
 (segment (start 70.6 157.084172) (end 70.6 152.6) (width 0.5) (layer "B.Cu") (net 19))
 (segment (start 67.584651 160.099521) (end 70.6 157.084172) (width 0.5) (layer "B.Cu") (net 19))
 (segment (start 57.825 155.44) (end 62.484521 160.099521) (width 0.5) (layer "B.Cu") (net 19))
 (segment (start 62.484521 160.099521) (end 67.584651 160.099521) (width 0.5) (layer "B.Cu") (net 19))
 (segment (start 69.9 144.7) (end 71.6 143) (width 0.5) (layer "B.Cu") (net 20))
 (segment (start 68.7 148.1) (end 69.9 146.9) (width 0.5) (layer "B.Cu") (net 20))
 (segment (start 66.339123 152.849511) (end 67.211855 152.849511) (width 0.5) (layer "B.Cu") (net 20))
 (segment (start 71.6 143) (end 73.6 143) (width 0.5) (layer "B.Cu") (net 20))
 (segment (start 67.211855 152.849511) (end 68.7 151.361366) (width 0.5) (layer "B.Cu") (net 20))
 (segment (start 69.9 146.9) (end 69.9 144.7) (width 0.5) (layer "B.Cu") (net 20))
 (segment (start 64.175 155.44) (end 64.175 155.013634) (width 0.5) (layer "B.Cu") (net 20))
 (segment (start 68.7 151.361366) (end 68.7 148.1) (width 0.5) (layer "B.Cu") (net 20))
 (segment (start 64.175 155.013634) (end 66.339123 152.849511) (width 0.5) (layer "B.Cu") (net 20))
 (segment (start 67.465 153.42) (end 67.465 153.336688) (width 0.5) (layer "F.Cu") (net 21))
 (segment (start 67.465 153.336688) (end 69.5 151.301688) (width 0.5) (layer "F.Cu") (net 21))
 (segment (start 66.715 154.17) (end 67.465 153.42) (width 0.5) (layer "F.Cu") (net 21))
 (segment (start 69.5 151.301688) (end 69.5 149.4) (width 0.5) (layer "F.Cu") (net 21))
 (via (at 69.5 149.4) (size 0.55) (drill 0.3) (layers "F.Cu" "B.Cu") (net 21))
 (segment (start 72.95 147.7) (end 73.65 147) (width 0.5) (layer "B.Cu") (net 21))
 (segment (start 69.5 149.175386) (end 70.975386 147.7) (width 0.5) (layer "B.Cu") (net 21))
 (segment (start 69.5 149.4) (end 69.5 149.175386) (width 0.5) (layer "B.Cu") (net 21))
 (segment (start 70.975386 147.7) (end 72.95 147.7) (width 0.5) (layer "B.Cu") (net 21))
 (segment (start 57.254172 157) (end 55.854172 155.6) (width 0.5) (layer "F.Cu") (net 22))
 (segment (start 53.775 155.6) (end 53.125 154.95) (width 0.5) (layer "F.Cu") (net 22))
 (segment (start 67.924521 155.900479) (end 65.599521 155.900479) (width 0.5) (layer "F.Cu") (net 22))
 (segment (start 55.854172 155.6) (end 53.775 155.6) (width 0.5) (layer "F.Cu") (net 22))
 (segment (start 65.599521 155.900479) (end 64.5 157) (width 0.5) (layer "F.Cu") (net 22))
 (segment (start 64.5 157) (end 57.254172 157) (width 0.5) (layer "F.Cu") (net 22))
 (segment (start 68.875 154.95) (end 70.325 156.4) (width 0.5) (layer "F.Cu") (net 22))
 (segment (start 70.325 156.4) (end 71.9375 156.4) (width 0.5) (layer "F.Cu") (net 22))
 (segment (start 71.9375 156.4) (end 72.3 156.7625) (width 0.5) (layer "F.Cu") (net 22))
 (segment (start 68.875 154.95) (end 67.924521 155.900479) (width 0.5) (layer "F.Cu") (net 22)))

